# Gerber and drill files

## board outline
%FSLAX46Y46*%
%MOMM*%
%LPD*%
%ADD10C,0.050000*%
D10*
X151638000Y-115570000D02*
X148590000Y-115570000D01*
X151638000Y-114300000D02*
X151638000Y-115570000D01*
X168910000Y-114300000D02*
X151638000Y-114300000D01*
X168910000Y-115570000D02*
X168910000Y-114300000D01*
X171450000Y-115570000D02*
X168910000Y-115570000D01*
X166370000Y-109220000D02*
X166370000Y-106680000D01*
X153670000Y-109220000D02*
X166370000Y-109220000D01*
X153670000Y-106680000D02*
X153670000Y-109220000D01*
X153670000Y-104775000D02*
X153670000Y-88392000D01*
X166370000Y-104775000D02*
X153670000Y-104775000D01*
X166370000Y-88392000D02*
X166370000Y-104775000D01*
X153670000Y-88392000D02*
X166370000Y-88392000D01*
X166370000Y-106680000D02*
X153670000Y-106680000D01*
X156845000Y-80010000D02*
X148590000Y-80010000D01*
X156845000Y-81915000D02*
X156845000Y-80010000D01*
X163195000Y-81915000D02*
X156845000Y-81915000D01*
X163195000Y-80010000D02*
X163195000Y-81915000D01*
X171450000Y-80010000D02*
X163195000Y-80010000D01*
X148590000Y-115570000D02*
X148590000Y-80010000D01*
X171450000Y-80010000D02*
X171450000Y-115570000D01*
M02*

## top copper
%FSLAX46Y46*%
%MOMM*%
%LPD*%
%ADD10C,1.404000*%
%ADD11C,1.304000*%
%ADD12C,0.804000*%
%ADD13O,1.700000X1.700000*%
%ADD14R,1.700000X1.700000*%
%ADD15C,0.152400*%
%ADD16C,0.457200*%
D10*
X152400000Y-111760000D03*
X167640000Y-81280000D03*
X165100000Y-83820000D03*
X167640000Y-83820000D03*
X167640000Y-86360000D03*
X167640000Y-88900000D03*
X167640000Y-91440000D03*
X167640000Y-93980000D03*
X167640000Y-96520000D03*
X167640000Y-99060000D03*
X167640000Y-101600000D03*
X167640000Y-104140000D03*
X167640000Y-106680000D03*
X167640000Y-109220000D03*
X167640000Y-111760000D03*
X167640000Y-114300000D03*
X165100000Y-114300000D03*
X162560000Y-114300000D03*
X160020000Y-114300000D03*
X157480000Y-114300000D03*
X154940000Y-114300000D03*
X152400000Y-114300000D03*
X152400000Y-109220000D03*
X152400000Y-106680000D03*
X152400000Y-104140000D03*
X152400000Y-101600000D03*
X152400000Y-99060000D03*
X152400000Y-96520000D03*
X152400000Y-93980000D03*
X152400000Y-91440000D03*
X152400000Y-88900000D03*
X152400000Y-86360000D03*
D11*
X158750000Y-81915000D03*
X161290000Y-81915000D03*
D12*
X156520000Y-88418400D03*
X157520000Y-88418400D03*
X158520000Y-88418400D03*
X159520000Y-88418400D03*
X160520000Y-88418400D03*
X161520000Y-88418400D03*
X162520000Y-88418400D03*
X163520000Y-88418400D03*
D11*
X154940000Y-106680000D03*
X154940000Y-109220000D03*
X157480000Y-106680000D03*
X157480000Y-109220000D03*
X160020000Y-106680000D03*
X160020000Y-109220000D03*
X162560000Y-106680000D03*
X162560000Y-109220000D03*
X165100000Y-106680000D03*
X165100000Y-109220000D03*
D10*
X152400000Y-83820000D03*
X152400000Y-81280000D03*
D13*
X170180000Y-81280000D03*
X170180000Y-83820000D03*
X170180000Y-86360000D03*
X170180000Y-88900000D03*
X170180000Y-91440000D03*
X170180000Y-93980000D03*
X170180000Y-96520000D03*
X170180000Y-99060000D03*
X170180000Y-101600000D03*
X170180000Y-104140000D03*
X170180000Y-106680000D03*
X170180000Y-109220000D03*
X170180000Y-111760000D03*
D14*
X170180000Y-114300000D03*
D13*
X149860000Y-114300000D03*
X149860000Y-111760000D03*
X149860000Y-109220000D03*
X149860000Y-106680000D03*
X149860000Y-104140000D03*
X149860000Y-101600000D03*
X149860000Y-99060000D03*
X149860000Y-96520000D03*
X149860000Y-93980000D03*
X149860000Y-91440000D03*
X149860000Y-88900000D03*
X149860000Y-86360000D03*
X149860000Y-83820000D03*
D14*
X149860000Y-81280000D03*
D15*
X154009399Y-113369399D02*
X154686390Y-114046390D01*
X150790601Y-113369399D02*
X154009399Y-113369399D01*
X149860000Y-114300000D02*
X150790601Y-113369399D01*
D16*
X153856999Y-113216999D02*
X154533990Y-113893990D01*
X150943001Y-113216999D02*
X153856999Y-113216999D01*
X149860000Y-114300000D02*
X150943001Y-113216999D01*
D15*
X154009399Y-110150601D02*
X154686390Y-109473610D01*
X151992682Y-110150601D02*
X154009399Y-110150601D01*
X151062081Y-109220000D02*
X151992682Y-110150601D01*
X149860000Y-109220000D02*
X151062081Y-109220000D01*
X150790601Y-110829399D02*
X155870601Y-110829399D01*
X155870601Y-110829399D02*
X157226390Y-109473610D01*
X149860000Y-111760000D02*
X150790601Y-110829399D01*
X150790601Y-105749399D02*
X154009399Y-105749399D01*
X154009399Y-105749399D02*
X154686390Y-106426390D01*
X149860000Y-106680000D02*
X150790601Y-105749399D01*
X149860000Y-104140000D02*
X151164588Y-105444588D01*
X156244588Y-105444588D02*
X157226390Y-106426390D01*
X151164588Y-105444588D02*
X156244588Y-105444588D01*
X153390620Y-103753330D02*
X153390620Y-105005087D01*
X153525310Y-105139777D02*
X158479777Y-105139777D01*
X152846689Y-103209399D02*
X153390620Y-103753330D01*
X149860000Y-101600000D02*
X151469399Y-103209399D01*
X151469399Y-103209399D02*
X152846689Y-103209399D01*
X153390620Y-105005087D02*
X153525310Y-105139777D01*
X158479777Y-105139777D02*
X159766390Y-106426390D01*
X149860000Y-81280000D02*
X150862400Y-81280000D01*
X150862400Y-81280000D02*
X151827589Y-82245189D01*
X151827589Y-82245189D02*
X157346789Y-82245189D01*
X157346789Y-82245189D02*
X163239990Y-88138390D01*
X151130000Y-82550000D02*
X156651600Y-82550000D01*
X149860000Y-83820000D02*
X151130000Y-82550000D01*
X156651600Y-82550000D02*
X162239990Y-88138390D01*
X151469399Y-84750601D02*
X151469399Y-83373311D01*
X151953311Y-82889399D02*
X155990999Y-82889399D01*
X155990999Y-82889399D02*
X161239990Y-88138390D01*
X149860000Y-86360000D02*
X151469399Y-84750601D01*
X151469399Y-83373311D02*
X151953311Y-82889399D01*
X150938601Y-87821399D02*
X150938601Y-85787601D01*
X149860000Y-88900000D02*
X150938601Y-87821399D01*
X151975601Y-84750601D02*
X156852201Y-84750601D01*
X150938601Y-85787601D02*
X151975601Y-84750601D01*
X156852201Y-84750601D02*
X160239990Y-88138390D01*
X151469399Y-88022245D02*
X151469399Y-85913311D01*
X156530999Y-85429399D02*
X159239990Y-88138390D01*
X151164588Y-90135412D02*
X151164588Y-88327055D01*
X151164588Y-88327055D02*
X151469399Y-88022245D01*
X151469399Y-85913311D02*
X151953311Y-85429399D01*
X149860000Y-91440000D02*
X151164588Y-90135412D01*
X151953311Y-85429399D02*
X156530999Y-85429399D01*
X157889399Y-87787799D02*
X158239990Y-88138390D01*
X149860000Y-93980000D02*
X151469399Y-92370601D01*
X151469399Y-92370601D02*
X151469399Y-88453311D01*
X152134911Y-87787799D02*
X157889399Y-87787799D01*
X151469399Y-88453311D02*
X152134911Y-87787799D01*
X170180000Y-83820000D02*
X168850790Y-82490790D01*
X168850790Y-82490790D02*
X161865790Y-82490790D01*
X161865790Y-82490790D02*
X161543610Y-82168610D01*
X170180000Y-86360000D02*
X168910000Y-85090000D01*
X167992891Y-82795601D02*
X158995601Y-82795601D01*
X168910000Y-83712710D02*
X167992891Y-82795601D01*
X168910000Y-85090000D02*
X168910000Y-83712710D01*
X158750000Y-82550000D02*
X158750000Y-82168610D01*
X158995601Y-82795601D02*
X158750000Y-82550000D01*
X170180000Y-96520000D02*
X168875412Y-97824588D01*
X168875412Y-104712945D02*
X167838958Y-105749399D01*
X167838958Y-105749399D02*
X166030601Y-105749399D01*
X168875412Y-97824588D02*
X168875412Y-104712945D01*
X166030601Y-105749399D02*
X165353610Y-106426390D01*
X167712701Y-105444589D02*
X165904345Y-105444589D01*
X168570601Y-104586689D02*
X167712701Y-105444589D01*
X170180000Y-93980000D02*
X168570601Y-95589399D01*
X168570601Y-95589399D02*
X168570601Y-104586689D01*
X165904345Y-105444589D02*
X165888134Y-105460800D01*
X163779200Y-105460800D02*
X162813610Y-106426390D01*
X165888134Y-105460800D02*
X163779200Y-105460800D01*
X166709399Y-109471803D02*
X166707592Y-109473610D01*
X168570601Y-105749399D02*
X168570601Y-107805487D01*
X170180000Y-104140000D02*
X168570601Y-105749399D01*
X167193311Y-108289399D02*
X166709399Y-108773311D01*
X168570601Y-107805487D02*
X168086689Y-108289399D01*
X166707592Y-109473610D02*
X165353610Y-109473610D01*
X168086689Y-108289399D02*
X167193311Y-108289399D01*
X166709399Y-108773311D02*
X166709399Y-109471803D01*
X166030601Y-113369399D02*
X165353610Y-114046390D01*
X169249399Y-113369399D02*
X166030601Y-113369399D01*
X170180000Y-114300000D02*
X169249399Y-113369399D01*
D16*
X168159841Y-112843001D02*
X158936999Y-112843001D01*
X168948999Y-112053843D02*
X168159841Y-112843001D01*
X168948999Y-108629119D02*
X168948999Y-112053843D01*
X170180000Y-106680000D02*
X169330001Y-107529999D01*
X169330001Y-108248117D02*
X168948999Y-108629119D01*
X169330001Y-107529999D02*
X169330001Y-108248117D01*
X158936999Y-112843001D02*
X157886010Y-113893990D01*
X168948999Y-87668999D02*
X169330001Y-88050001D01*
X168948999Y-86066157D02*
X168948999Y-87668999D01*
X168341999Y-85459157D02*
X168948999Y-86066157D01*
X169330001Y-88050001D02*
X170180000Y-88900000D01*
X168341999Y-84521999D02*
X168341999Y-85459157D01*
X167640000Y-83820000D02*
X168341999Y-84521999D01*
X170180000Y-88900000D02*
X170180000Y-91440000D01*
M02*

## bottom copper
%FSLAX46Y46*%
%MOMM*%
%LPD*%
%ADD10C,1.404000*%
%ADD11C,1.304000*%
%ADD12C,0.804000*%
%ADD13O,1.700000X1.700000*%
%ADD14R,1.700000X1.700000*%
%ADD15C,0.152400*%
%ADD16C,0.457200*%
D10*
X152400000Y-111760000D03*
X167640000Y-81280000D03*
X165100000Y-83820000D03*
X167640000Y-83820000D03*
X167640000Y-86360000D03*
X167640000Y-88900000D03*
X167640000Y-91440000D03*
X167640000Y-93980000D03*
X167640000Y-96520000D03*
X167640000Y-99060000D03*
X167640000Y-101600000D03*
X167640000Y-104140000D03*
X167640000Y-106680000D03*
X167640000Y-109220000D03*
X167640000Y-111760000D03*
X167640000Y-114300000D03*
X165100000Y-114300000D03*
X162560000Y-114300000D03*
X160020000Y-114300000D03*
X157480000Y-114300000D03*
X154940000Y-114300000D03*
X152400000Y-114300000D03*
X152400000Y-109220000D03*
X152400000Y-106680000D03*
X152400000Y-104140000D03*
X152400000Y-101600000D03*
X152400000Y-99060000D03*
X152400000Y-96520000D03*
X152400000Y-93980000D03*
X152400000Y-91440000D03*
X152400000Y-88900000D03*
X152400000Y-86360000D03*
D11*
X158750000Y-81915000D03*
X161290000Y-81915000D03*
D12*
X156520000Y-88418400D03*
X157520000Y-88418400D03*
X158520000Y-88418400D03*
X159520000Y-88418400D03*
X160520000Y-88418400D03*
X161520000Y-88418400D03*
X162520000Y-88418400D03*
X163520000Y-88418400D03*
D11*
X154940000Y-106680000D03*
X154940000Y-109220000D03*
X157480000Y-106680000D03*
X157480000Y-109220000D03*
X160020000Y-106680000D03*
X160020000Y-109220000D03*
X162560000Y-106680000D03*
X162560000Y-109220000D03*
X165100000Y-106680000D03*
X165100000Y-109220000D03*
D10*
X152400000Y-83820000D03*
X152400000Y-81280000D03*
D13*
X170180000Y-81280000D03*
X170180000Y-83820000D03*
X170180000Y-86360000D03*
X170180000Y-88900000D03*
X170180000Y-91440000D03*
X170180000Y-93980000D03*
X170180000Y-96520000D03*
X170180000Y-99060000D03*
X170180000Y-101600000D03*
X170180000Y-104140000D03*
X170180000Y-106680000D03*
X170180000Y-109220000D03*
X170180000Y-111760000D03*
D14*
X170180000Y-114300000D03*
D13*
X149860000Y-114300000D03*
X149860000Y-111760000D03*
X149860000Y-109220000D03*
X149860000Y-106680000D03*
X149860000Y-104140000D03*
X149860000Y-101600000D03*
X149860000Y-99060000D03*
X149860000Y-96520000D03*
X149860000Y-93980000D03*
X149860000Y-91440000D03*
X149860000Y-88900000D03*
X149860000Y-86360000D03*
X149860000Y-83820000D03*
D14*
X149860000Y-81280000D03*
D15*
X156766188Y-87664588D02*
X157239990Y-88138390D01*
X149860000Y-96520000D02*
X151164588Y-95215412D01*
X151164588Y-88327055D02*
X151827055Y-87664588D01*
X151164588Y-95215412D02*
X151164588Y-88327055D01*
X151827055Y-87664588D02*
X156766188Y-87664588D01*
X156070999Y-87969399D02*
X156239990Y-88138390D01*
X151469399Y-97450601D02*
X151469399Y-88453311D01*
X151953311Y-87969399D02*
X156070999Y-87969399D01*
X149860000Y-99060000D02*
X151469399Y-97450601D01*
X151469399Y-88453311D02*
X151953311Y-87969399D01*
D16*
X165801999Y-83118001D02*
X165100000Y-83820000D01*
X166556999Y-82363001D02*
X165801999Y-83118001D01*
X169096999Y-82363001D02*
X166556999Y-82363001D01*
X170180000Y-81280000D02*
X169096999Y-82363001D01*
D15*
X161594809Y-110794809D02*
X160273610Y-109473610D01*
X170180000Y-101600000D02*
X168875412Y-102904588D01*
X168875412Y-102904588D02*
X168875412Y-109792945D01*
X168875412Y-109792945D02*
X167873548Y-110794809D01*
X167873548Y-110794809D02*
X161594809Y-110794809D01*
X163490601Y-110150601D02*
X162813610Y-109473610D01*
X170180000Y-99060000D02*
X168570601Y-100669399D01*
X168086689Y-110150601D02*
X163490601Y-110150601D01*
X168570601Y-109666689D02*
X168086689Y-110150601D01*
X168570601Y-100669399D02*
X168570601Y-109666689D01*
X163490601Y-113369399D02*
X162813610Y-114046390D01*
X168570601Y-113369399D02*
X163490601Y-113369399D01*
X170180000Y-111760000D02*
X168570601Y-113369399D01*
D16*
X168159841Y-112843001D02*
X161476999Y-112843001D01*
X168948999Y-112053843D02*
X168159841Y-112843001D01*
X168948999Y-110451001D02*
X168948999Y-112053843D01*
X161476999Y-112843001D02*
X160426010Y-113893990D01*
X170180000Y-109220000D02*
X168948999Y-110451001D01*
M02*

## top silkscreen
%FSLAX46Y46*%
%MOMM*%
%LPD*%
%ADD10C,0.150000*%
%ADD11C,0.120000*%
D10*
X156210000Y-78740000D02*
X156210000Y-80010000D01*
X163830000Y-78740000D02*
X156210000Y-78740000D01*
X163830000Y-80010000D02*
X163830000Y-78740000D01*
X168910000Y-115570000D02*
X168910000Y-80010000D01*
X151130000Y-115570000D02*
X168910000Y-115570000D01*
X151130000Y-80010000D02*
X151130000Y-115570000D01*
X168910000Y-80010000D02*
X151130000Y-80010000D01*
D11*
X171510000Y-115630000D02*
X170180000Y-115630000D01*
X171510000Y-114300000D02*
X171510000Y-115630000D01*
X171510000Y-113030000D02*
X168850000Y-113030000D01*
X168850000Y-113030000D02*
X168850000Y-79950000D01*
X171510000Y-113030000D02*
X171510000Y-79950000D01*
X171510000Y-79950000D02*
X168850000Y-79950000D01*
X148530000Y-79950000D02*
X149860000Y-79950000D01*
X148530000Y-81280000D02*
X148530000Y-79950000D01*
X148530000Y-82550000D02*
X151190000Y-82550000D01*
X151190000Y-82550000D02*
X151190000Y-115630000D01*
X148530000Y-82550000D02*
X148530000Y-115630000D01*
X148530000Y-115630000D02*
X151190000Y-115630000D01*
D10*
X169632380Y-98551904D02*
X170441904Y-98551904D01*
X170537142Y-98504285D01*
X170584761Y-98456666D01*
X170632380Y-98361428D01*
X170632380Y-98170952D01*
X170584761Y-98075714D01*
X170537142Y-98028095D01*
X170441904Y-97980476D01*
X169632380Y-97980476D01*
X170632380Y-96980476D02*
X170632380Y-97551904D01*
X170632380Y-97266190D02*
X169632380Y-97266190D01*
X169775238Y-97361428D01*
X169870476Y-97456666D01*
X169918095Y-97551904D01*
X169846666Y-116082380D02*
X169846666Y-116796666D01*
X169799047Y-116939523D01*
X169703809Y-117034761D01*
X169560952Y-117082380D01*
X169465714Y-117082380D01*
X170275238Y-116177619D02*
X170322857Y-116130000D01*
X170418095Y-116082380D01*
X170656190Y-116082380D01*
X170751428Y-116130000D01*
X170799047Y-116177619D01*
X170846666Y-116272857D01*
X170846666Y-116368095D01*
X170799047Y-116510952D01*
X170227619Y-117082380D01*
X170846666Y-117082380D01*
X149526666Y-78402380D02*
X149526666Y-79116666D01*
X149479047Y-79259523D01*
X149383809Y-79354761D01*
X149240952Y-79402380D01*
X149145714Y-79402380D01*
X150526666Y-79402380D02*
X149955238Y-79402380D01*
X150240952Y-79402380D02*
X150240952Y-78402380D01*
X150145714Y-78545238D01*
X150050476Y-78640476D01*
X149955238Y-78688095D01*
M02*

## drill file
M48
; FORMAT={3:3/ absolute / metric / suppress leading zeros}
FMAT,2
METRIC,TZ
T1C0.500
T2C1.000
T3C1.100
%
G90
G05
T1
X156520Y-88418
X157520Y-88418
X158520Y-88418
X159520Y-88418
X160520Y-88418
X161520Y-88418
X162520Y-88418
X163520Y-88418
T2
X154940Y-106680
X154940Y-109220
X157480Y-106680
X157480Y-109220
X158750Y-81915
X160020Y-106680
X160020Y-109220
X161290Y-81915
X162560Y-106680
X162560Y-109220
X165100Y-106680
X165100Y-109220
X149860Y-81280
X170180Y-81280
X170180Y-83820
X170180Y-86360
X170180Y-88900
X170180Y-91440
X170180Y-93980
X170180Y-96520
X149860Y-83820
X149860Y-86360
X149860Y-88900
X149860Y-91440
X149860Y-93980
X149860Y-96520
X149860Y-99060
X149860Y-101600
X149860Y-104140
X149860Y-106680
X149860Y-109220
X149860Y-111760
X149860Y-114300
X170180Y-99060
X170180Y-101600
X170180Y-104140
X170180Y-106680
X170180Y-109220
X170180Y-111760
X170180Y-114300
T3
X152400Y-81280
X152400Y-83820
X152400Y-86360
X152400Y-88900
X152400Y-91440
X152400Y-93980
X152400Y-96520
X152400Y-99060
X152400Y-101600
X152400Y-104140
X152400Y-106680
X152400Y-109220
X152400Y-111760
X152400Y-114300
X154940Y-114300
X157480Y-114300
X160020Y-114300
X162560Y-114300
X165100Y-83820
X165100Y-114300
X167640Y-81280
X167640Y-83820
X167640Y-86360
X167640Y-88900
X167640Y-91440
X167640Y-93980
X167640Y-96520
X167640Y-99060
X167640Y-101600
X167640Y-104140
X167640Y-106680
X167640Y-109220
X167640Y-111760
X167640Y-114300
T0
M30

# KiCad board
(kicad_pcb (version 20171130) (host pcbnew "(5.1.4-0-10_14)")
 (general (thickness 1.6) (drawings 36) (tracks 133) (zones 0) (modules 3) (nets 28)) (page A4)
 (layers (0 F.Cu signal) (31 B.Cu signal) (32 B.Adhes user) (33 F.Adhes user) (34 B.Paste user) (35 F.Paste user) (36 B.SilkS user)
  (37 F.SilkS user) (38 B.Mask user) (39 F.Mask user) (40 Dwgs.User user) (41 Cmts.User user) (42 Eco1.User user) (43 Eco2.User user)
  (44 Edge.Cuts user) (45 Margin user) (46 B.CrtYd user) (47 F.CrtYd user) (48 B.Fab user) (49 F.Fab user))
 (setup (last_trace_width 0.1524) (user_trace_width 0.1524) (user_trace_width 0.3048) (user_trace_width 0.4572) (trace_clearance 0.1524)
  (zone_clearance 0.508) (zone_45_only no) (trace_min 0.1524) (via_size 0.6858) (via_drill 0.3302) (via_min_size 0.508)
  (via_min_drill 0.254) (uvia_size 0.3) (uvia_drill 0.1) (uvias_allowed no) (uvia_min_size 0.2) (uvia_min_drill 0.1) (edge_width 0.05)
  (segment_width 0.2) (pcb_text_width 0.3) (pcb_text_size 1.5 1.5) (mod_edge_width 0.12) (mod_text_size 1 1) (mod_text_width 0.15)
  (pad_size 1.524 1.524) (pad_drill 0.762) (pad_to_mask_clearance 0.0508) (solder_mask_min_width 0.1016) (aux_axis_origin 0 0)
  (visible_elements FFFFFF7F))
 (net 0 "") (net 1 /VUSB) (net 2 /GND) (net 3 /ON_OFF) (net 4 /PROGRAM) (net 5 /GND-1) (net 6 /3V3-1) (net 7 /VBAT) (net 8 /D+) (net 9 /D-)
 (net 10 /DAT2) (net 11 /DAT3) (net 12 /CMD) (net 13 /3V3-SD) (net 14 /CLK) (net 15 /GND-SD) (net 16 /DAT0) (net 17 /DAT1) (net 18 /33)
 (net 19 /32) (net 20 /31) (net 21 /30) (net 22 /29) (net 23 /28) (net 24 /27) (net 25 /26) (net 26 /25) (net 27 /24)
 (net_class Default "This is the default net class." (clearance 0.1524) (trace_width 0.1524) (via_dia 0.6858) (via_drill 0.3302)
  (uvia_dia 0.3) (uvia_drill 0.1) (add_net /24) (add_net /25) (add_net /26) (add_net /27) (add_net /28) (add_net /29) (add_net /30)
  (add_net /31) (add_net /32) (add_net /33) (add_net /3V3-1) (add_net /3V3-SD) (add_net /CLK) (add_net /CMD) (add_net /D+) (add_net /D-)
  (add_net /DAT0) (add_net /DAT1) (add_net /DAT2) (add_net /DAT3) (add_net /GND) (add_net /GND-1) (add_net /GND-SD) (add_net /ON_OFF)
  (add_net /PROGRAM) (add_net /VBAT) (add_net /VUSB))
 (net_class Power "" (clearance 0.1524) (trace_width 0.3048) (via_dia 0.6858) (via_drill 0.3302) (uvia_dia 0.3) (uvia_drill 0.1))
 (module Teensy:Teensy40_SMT (layer F.Cu) (at 160.02 97.79 270)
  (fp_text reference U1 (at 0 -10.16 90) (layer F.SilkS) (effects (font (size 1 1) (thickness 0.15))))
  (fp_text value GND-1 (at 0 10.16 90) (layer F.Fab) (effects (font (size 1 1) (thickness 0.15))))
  (fp_line (start -19.05 3.81) (end -17.78 3.81) (layer F.SilkS) (width 0.15))
  (fp_line (start -19.05 -3.81) (end -19.05 3.81) (layer F.SilkS) (width 0.15))
  (fp_line (start -17.78 -3.81) (end -19.05 -3.81) (layer F.SilkS) (width 0.15))
  (fp_line (start 17.78 -8.89) (end -17.78 -8.89) (layer F.SilkS) (width 0.15))
  (fp_line (start 17.78 8.89) (end 17.78 -8.89) (layer F.SilkS) (width 0.15))
  (fp_line (start -17.78 8.89) (end 17.78 8.89) (layer F.SilkS) (width 0.15))
  (fp_line (start -17.78 -8.89) (end -17.78 8.89) (layer F.SilkS) (width 0.15))
  (pad 13 thru_hole circle (at 13.97 7.62 270) (size 1.404 1.404) (drill 1.1) (layers *.Cu *.Mask))
  (pad 33 thru_hole circle (at -16.51 -7.62 270) (size 1.404 1.404) (drill 1.1) (layers *.Cu *.Mask))
  (pad 34 thru_hole circle (at -13.97 -5.08 270) (size 1.404 1.404) (drill 1.1) (layers *.Cu *.Mask) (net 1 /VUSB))
  (pad 32 thru_hole circle (at -13.97 -7.62 270) (size 1.404 1.404) (drill 1.1) (layers *.Cu *.Mask) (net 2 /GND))
  (pad 31 thru_hole circle (at -11.43 -7.62 270) (size 1.404 1.404) (drill 1.1) (layers *.Cu *.Mask))
  (pad 30 thru_hole circle (at -8.89 -7.62 270) (size 1.404 1.404) (drill 1.1) (layers *.Cu *.Mask))
  (pad 29 thru_hole circle (at -6.35 -7.62 270) (size 1.404 1.404) (drill 1.1) (layers *.Cu *.Mask))
  (pad 28 thru_hole circle (at -3.81 -7.62 270) (size 1.404 1.404) (drill 1.1) (layers *.Cu *.Mask))
  (pad 27 thru_hole circle (at -1.27 -7.62 270) (size 1.404 1.404) (drill 1.1) (layers *.Cu *.Mask))
  (pad 26 thru_hole circle (at 1.27 -7.62 270) (size 1.404 1.404) (drill 1.1) (layers *.Cu *.Mask))
  (pad 25 thru_hole circle (at 3.81 -7.62 270) (size 1.404 1.404) (drill 1.1) (layers *.Cu *.Mask))
  (pad 24 thru_hole circle (at 6.35 -7.62 270) (size 1.404 1.404) (drill 1.1) (layers *.Cu *.Mask))
  (pad 23 thru_hole circle (at 8.89 -7.62 270) (size 1.404 1.404) (drill 1.1) (layers *.Cu *.Mask))
  (pad 22 thru_hole circle (at 11.43 -7.62 270) (size 1.404 1.404) (drill 1.1) (layers *.Cu *.Mask))
  (pad 21 thru_hole circle (at 13.97 -7.62 270) (size 1.404 1.404) (drill 1.1) (layers *.Cu *.Mask))
  (pad 20 thru_hole circle (at 16.51 -7.62 270) (size 1.404 1.404) (drill 1.1) (layers *.Cu *.Mask))
  (pad 19 thru_hole circle (at 16.51 -5.08 270) (size 1.404 1.404) (drill 1.1) (layers *.Cu *.Mask) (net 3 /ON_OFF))
  (pad 18 thru_hole circle (at 16.51 -2.54 270) (size 1.404 1.404) (drill 1.1) (layers *.Cu *.Mask) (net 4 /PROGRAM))
  (pad 17 thru_hole circle (at 16.51 0 270) (size 1.404 1.404) (drill 1.1) (layers *.Cu *.Mask) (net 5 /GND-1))
  (pad 16 thru_hole circle (at 16.51 2.54 270) (size 1.404 1.404) (drill 1.1) (layers *.Cu *.Mask) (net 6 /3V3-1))
  (pad 15 thru_hole circle (at 16.51 5.08 270) (size 1.404 1.404) (drill 1.1) (layers *.Cu *.Mask) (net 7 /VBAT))
  (pad 14 thru_hole circle (at 16.51 7.62 270) (size 1.404 1.404) (drill 1.1) (layers *.Cu *.Mask))
  (pad 12 thru_hole circle (at 11.43 7.62 270) (size 1.404 1.404) (drill 1.1) (layers *.Cu *.Mask))
  (pad 11 thru_hole circle (at 8.89 7.62 270) (size 1.404 1.404) (drill 1.1) (layers *.Cu *.Mask))
  (pad 10 thru_hole circle (at 6.35 7.62 270) (size 1.404 1.404) (drill 1.1) (layers *.Cu *.Mask))
  (pad 9 thru_hole circle (at 3.81 7.62 270) (size 1.404 1.404) (drill 1.1) (layers *.Cu *.Mask))
  (pad 8 thru_hole circle (at 1.27 7.62 270) (size 1.404 1.404) (drill 1.1) (layers *.Cu *.Mask))
  (pad 7 thru_hole circle (at -1.27 7.62 270) (size 1.404 1.404) (drill 1.1) (layers *.Cu *.Mask))
  (pad 6 thru_hole circle (at -3.81 7.62 270) (size 1.404 1.404) (drill 1.1) (layers *.Cu *.Mask))
  (pad 5 thru_hole circle (at -6.35 7.62 270) (size 1.404 1.404) (drill 1.1) (layers *.Cu *.Mask))
  (pad 4 thru_hole circle (at -8.89 7.62 270) (size 1.404 1.404) (drill 1.1) (layers *.Cu *.Mask))
  (pad 3 thru_hole circle (at -11.43 7.62 270) (size 1.404 1.404) (drill 1.1) (layers *.Cu *.Mask))
  (pad 54 thru_hole circle (at -15.875 1.27 270) (size 1.304 1.304) (drill 1) (layers *.Cu *.Mask) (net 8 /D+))
  (pad 53 thru_hole circle (at -15.875 -1.27 270) (size 1.304 1.304) (drill 1) (layers *.Cu *.Mask) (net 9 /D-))
  (pad 52 thru_hole circle (at -9.3716 3.5 270) (size 0.804 0.804) (drill 0.5) (layers *.Cu *.Mask) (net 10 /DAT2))
  (pad 51 thru_hole circle (at -9.3716 2.5 270) (size 0.804 0.804) (drill 0.5) (layers *.Cu *.Mask) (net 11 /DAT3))
  (pad 50 thru_hole circle (at -9.3716 1.5 270) (size 0.804 0.804) (drill 0.5) (layers *.Cu *.Mask) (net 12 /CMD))
  (pad 49 thru_hole circle (at -9.3716 0.5 270) (size 0.804 0.804) (drill 0.5) (layers *.Cu *.Mask) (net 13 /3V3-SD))
  (pad 48 thru_hole circle (at -9.3716 -0.5 270) (size 0.804 0.804) (drill 0.5) (layers *.Cu *.Mask) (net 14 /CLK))
  (pad 47 thru_hole circle (at -9.3716 -1.5 270) (size 0.804 0.804) (drill 0.5) (layers *.Cu *.Mask) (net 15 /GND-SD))
  (pad 46 thru_hole circle (at -9.3716 -2.5 270) (size 0.804 0.804) (drill 0.5) (layers *.Cu *.Mask) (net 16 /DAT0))
  (pad 45 thru_hole circle (at -9.3716 -3.5 270) (size 0.804 0.804) (drill 0.5) (layers *.Cu *.Mask) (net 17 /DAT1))
  (pad 44 thru_hole circle (at 8.89 5.08 270) (size 1.304 1.304) (drill 1) (layers *.Cu *.Mask) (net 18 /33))
  (pad 43 thru_hole circle (at 11.43 5.08 270) (size 1.304 1.304) (drill 1) (layers *.Cu *.Mask) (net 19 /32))
  (pad 42 thru_hole circle (at 8.89 2.54 270) (size 1.304 1.304) (drill 1) (layers *.Cu *.Mask) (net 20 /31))
  (pad 41 thru_hole circle (at 11.43 2.54 270) (size 1.304 1.304) (drill 1) (layers *.Cu *.Mask) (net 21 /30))
  (pad 40 thru_hole circle (at 8.89 0 270) (size 1.304 1.304) (drill 1) (layers *.Cu *.Mask) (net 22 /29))
  (pad 39 thru_hole circle (at 11.43 0 270) (size 1.304 1.304) (drill 1) (layers *.Cu *.Mask) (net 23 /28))
  (pad 38 thru_hole circle (at 8.89 -2.54 270) (size 1.304 1.304) (drill 1) (layers *.Cu *.Mask) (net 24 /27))
  (pad 37 thru_hole circle (at 11.43 -2.54 270) (size 1.304 1.304) (drill 1) (layers *.Cu *.Mask) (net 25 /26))
  (pad 36 thru_hole circle (at 8.89 -5.08 270) (size 1.304 1.304) (drill 1) (layers *.Cu *.Mask) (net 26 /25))
  (pad 35 thru_hole circle (at 11.43 -5.08 270) (size 1.304 1.304) (drill 1) (layers *.Cu *.Mask) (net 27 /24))
  (pad 2 thru_hole circle (at -13.97 7.62 270) (size 1.404 1.404) (drill 1.1) (layers *.Cu *.Mask))
  (pad 1 thru_hole circle (at -16.51 7.62 270) (size 1.404 1.404) (drill 1.1) (layers *.Cu *.Mask)))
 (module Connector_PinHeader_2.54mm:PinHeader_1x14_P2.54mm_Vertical (layer F.Cu) (at 170.18 114.3 180)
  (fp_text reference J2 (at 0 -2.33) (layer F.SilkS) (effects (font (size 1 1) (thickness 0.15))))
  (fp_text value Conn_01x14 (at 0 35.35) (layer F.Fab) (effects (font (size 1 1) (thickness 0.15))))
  (fp_line (start -1.33 -1.33) (end 0 -1.33) (layer F.SilkS) (width 0.12))
  (fp_line (start -1.33 0) (end -1.33 -1.33) (layer F.SilkS) (width 0.12))
  (fp_line (start -1.33 1.27) (end 1.33 1.27) (layer F.SilkS) (width 0.12))
  (fp_line (start 1.33 1.27) (end 1.33 34.35) (layer F.SilkS) (width 0.12))
  (fp_line (start -1.33 1.27) (end -1.33 34.35) (layer F.SilkS) (width 0.12))
  (fp_line (start -1.33 34.35) (end 1.33 34.35) (layer F.SilkS) (width 0.12))
  (pad 14 thru_hole oval (at 0 33.02 180) (size 1.7 1.7) (drill 1) (layers *.Cu *.Mask) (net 1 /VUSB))
  (pad 13 thru_hole oval (at 0 30.48 180) (size 1.7 1.7) (drill 1) (layers *.Cu *.Mask) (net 9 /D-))
  (pad 12 thru_hole oval (at 0 27.94 180) (size 1.7 1.7) (drill 1) (layers *.Cu *.Mask) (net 8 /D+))
  (pad 11 thru_hole oval (at 0 25.4 180) (size 1.7 1.7) (drill 1) (layers *.Cu *.Mask) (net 2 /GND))
  (pad 10 thru_hole oval (at 0 22.86 180) (size 1.7 1.7) (drill 1) (layers *.Cu *.Mask) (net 2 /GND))
  (pad 9 thru_hole oval (at 0 20.32 180) (size 1.7 1.7) (drill 1) (layers *.Cu *.Mask) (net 24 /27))
  (pad 8 thru_hole oval (at 0 17.78 180) (size 1.7 1.7) (drill 1) (layers *.Cu *.Mask) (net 26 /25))
  (pad 7 thru_hole oval (at 0 15.24 180) (size 1.7 1.7) (drill 1) (layers *.Cu *.Mask) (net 25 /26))
  (pad 6 thru_hole oval (at 0 12.7 180) (size 1.7 1.7) (drill 1) (layers *.Cu *.Mask) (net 23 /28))
  (pad 5 thru_hole oval (at 0 10.16 180) (size 1.7 1.7) (drill 1) (layers *.Cu *.Mask) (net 27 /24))
  (pad 4 thru_hole oval (at 0 7.62 180) (size 1.7 1.7) (drill 1) (layers *.Cu *.Mask) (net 6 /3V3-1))
  (pad 3 thru_hole oval (at 0 5.08 180) (size 1.7 1.7) (drill 1) (layers *.Cu *.Mask) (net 5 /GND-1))
  (pad 2 thru_hole oval (at 0 2.54 180) (size 1.7 1.7) (drill 1) (layers *.Cu *.Mask) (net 4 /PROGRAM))
  (pad 1 thru_hole rect (at 0 0 180) (size 1.7 1.7) (drill 1) (layers *.Cu *.Mask) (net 3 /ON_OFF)))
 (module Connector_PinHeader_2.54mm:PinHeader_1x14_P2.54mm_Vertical (layer F.Cu) (at 149.86 81.28)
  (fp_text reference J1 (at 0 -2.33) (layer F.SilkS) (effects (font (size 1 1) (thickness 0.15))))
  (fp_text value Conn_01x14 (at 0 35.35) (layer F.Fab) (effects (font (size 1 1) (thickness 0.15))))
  (fp_line (start -1.33 -1.33) (end 0 -1.33) (layer F.SilkS) (width 0.12))
  (fp_line (start -1.33 0) (end -1.33 -1.33) (layer F.SilkS) (width 0.12))
  (fp_line (start -1.33 1.27) (end 1.33 1.27) (layer F.SilkS) (width 0.12))
  (fp_line (start 1.33 1.27) (end 1.33 34.35) (layer F.SilkS) (width 0.12))
  (fp_line (start -1.33 1.27) (end -1.33 34.35) (layer F.SilkS) (width 0.12))
  (fp_line (start -1.33 34.35) (end 1.33 34.35) (layer F.SilkS) (width 0.12))
  (pad 14 thru_hole oval (at 0 33.02) (size 1.7 1.7) (drill 1) (layers *.Cu *.Mask) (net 7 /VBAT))
  (pad 13 thru_hole oval (at 0 30.48) (size 1.7 1.7) (drill 1) (layers *.Cu *.Mask) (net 21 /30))
  (pad 12 thru_hole oval (at 0 27.94) (size 1.7 1.7) (drill 1) (layers *.Cu *.Mask) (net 19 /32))
  (pad 11 thru_hole oval (at 0 25.4) (size 1.7 1.7) (drill 1) (layers *.Cu *.Mask) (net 18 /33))
  (pad 10 thru_hole oval (at 0 22.86) (size 1.7 1.7) (drill 1) (layers *.Cu *.Mask) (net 20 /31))
  (pad 9 thru_hole oval (at 0 20.32) (size 1.7 1.7) (drill 1) (layers *.Cu *.Mask) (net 22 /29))
  (pad 8 thru_hole oval (at 0 17.78) (size 1.7 1.7) (drill 1) (layers *.Cu *.Mask) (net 10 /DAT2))
  (pad 7 thru_hole oval (at 0 15.24) (size 1.7 1.7) (drill 1) (layers *.Cu *.Mask) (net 11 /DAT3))
  (pad 6 thru_hole oval (at 0 12.7) (size 1.7 1.7) (drill 1) (layers *.Cu *.Mask) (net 12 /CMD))
  (pad 5 thru_hole oval (at 0 10.16) (size 1.7 1.7) (drill 1) (layers *.Cu *.Mask) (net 13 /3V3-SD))
  (pad 4 thru_hole oval (at 0 7.62) (size 1.7 1.7) (drill 1) (layers *.Cu *.Mask) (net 14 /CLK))
  (pad 3 thru_hole oval (at 0 5.08) (size 1.7 1.7) (drill 1) (layers *.Cu *.Mask) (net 15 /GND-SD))
  (pad 2 thru_hole oval (at 0 2.54) (size 1.7 1.7) (drill 1) (layers *.Cu *.Mask) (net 16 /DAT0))
  (pad 1 thru_hole rect (at 0 0) (size 1.7 1.7) (drill 1) (layers *.Cu *.Mask) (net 17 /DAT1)))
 (gr_line (start 151.638 115.57) (end 148.59 115.57) (layer Edge.Cuts) (width 0.05))
 (gr_line (start 151.638 114.3) (end 151.638 115.57) (layer Edge.Cuts) (width 0.05))
 (gr_line (start 168.91 114.3) (end 151.638 114.3) (layer Edge.Cuts) (width 0.05))
 (gr_line (start 168.91 115.57) (end 168.91 114.3) (layer Edge.Cuts) (width 0.05))
 (gr_line (start 171.45 115.57) (end 168.91 115.57) (layer Edge.Cuts) (width 0.05))
 (gr_line (start 166.37 109.22) (end 166.37 106.68) (layer Edge.Cuts) (width 0.05))
 (gr_line (start 153.67 109.22) (end 166.37 109.22) (layer Edge.Cuts) (width 0.05))
 (gr_line (start 153.67 106.68) (end 153.67 109.22) (layer Edge.Cuts) (width 0.05))
 (gr_line (start 153.67 104.775) (end 153.67 88.392) (layer Edge.Cuts) (width 0.05))
 (gr_line (start 166.37 104.775) (end 153.67 104.775) (layer Edge.Cuts) (width 0.05))
 (gr_line (start 166.37 88.392) (end 166.37 104.775) (layer Edge.Cuts) (width 0.05))
 (gr_line (start 153.67 88.392) (end 166.37 88.392) (layer Edge.Cuts) (width 0.05))
 (gr_line (start 166.37 106.68) (end 153.67 106.68) (layer Edge.Cuts) (width 0.05))
 (gr_line (start 156.845 80.01) (end 148.59 80.01) (layer Edge.Cuts) (width 0.05))
 (gr_line (start 156.845 81.915) (end 156.845 80.01) (layer Edge.Cuts) (width 0.05))
 (gr_line (start 163.195 81.915) (end 156.845 81.915) (layer Edge.Cuts) (width 0.05))
 (gr_line (start 163.195 80.01) (end 163.195 81.915) (layer Edge.Cuts) (width 0.05))
 (gr_line (start 171.45 80.01) (end 163.195 80.01) (layer Edge.Cuts) (width 0.05))
 (gr_line (start 148.59 115.57) (end 148.59 80.01) (layer Edge.Cuts) (width 0.05))
 (gr_line (start 171.45 80.01) (end 171.45 115.57) (layer Edge.Cuts) (width 0.05))
 (segment (start 154.009399 113.369399) (end 154.68639 114.04639) (width 0.1524) (layer F.Cu) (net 7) (status 20))
 (segment (start 150.790601 113.369399) (end 154.009399 113.369399) (width 0.1524) (layer F.Cu) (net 7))
 (segment (start 149.86 114.3) (end 150.790601 113.369399) (width 0.1524) (layer F.Cu) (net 7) (status 10))
 (segment (start 153.856999 113.216999) (end 154.53399 113.89399) (width 0.4572) (layer F.Cu) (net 7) (status 20))
 (segment (start 150.943001 113.216999) (end 153.856999 113.216999) (width 0.4572) (layer F.Cu) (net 7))
 (segment (start 149.86 114.3) (end 150.943001 113.216999) (width 0.4572) (layer F.Cu) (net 7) (status 10))
 (segment (start 154.009399 110.150601) (end 154.68639 109.47361) (width 0.1524) (layer F.Cu) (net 19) (status 20))
 (segment (start 151.992682 110.150601) (end 154.009399 110.150601) (width 0.1524) (layer F.Cu) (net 19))
 (segment (start 151.062081 109.22) (end 151.992682 110.150601) (width 0.1524) (layer F.Cu) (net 19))
 (segment (start 149.86 109.22) (end 151.062081 109.22) (width 0.1524) (layer F.Cu) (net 19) (status 10))
 (segment (start 150.790601 110.829399) (end 155.870601 110.829399) (width 0.1524) (layer F.Cu) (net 21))
 (segment (start 155.870601 110.829399) (end 157.22639 109.47361) (width 0.1524) (layer F.Cu) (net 21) (status 20))
 (segment (start 149.86 111.76) (end 150.790601 110.829399) (width 0.1524) (layer F.Cu) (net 21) (status 10))
 (segment (start 150.790601 105.749399) (end 154.009399 105.749399) (width 0.1524) (layer F.Cu) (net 18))
 (segment (start 154.009399 105.749399) (end 154.68639 106.42639) (width 0.1524) (layer F.Cu) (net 18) (status 20))
 (segment (start 149.86 106.68) (end 150.790601 105.749399) (width 0.1524) (layer F.Cu) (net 18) (status 10))
 (segment (start 149.86 104.14) (end 151.164588 105.444588) (width 0.1524) (layer F.Cu) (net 20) (status 10))
 (segment (start 156.244588 105.444588) (end 157.22639 106.42639) (width 0.1524) (layer F.Cu) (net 20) (status 20))
 (segment (start 151.164588 105.444588) (end 156.244588 105.444588) (width 0.1524) (layer F.Cu) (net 20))
 (segment (start 153.39062 103.75333) (end 153.39062 105.005087) (width 0.1524) (layer F.Cu) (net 22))
 (segment (start 153.52531 105.139777) (end 158.479777 105.139777) (width 0.1524) (layer F.Cu) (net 22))
 (segment (start 152.846689 103.209399) (end 153.39062 103.75333) (width 0.1524) (layer F.Cu) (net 22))
 (segment (start 149.86 101.6) (end 151.469399 103.209399) (width 0.1524) (layer F.Cu) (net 22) (status 10))
 (segment (start 151.469399 103.209399) (end 152.846689 103.209399) (width 0.1524) (layer F.Cu) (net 22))
 (segment (start 153.39062 105.005087) (end 153.52531 105.139777) (width 0.1524) (layer F.Cu) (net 22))
 (segment (start 158.479777 105.139777) (end 159.76639 106.42639) (width 0.1524) (layer F.Cu) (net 22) (status 20))
 (segment (start 149.86 81.28) (end 150.8624 81.28) (width 0.1524) (layer F.Cu) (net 17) (status 10))
 (segment (start 150.8624 81.28) (end 151.827589 82.245189) (width 0.1524) (layer F.Cu) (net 17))
 (segment (start 151.827589 82.245189) (end 157.346789 82.245189) (width 0.1524) (layer F.Cu) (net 17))
 (segment (start 157.346789 82.245189) (end 163.23999 88.13839) (width 0.1524) (layer F.Cu) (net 17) (status 20))
 (segment (start 151.13 82.55) (end 156.6516 82.55) (width 0.1524) (layer F.Cu) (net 16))
 (segment (start 149.86 83.82) (end 151.13 82.55) (width 0.1524) (layer F.Cu) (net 16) (status 10))
 (segment (start 156.6516 82.55) (end 162.23999 88.13839) (width 0.1524) (layer F.Cu) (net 16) (status 20))
 (segment (start 151.469399 84.750601) (end 151.469399 83.373311) (width 0.1524) (layer F.Cu) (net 15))
 (segment (start 151.953311 82.889399) (end 155.990999 82.889399) (width 0.1524) (layer F.Cu) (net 15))
 (segment (start 155.990999 82.889399) (end 161.23999 88.13839) (width 0.1524) (layer F.Cu) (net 15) (status 20))
 (segment (start 149.86 86.36) (end 151.469399 84.750601) (width 0.1524) (layer F.Cu) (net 15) (status 10))
 (segment (start 151.469399 83.373311) (end 151.953311 82.889399) (width 0.1524) (layer F.Cu) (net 15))
 (segment (start 150.938601 87.821399) (end 150.938601 85.787601) (width 0.1524) (layer F.Cu) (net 14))
 (segment (start 149.86 88.9) (end 150.938601 87.821399) (width 0.1524) (layer F.Cu) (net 14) (status 10))
 (segment (start 151.975601 84.750601) (end 156.852201 84.750601) (width 0.1524) (layer F.Cu) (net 14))
 (segment (start 150.938601 85.787601) (end 151.975601 84.750601) (width 0.1524) (layer F.Cu) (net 14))
 (segment (start 156.852201 84.750601) (end 160.23999 88.13839) (width 0.1524) (layer F.Cu) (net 14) (status 20))
 (segment (start 151.469399 88.022245) (end 151.469399 85.913311) (width 0.1524) (layer F.Cu) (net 13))
 (segment (start 156.530999 85.429399) (end 159.23999 88.13839) (width 0.1524) (layer F.Cu) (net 13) (status 20))
 (segment (start 151.164588 90.135412) (end 151.164588 88.327055) (width 0.1524) (layer F.Cu) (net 13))
 (segment (start 151.164588 88.327055) (end 151.469399 88.022245) (width 0.1524) (layer F.Cu) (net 13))
 (segment (start 151.469399 85.913311) (end 151.953311 85.429399) (width 0.1524) (layer F.Cu) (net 13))
 (segment (start 149.86 91.44) (end 151.164588 90.135412) (width 0.1524) (layer F.Cu) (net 13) (status 10))
 (segment (start 151.953311 85.429399) (end 156.530999 85.429399) (width 0.1524) (layer F.Cu) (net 13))
 (segment (start 157.889399 87.787799) (end 158.23999 88.13839) (width 0.1524) (layer F.Cu) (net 12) (status 20))
 (segment (start 149.86 93.98) (end 151.469399 92.370601) (width 0.1524) (layer F.Cu) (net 12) (status 10))
 (segment (start 151.469399 92.370601) (end 151.469399 88.453311) (width 0.1524) (layer F.Cu) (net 12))
 (segment (start 152.134911 87.787799) (end 157.889399 87.787799) (width 0.1524) (layer F.Cu) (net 12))
 (segment (start 151.469399 88.453311) (end 152.134911 87.787799) (width 0.1524) (layer F.Cu) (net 12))
 (segment (start 156.766188 87.664588) (end 157.23999 88.13839) (width 0.1524) (layer B.Cu) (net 11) (status 20))
 (segment (start 149.86 96.52) (end 151.164588 95.215412) (width 0.1524) (layer B.Cu) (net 11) (status 10))
 (segment (start 151.164588 88.327055) (end 151.827055 87.664588) (width 0.1524) (layer B.Cu) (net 11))
 (segment (start 151.164588 95.215412) (end 151.164588 88.327055) (width 0.1524) (layer B.Cu) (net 11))
 (segment (start 151.827055 87.664588) (end 156.766188 87.664588) (width 0.1524) (layer B.Cu) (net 11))
 (segment (start 156.070999 87.969399) (end 156.23999 88.13839) (width 0.1524) (layer B.Cu) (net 10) (status 20))
 (segment (start 151.469399 97.450601) (end 151.469399 88.453311) (width 0.1524) (layer B.Cu) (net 10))
 (segment (start 151.953311 87.969399) (end 156.070999 87.969399) (width 0.1524) (layer B.Cu) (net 10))
 (segment (start 149.86 99.06) (end 151.469399 97.450601) (width 0.1524) (layer B.Cu) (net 10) (status 10))
 (segment (start 151.469399 88.453311) (end 151.953311 87.969399) (width 0.1524) (layer B.Cu) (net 10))
 (segment (start 165.801999 83.118001) (end 165.1 83.82) (width 0.4572) (layer B.Cu) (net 1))
 (segment (start 166.556999 82.363001) (end 165.801999 83.118001) (width 0.4572) (layer B.Cu) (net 1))
 (segment (start 169.096999 82.363001) (end 166.556999 82.363001) (width 0.4572) (layer B.Cu) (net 1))
 (segment (start 170.18 81.28) (end 169.096999 82.363001) (width 0.4572) (layer B.Cu) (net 1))
 (segment (start 170.18 83.82) (end 168.85079 82.49079) (width 0.1524) (layer F.Cu) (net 9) (status 10))
 (segment (start 168.85079 82.49079) (end 161.86579 82.49079) (width 0.1524) (layer F.Cu) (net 9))
 (segment (start 161.86579 82.49079) (end 161.54361 82.16861) (width 0.1524) (layer F.Cu) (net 9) (status 20))
 (segment (start 170.18 86.36) (end 168.91 85.09) (width 0.1524) (layer F.Cu) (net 8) (status 10))
 (segment (start 167.992891 82.795601) (end 158.995601 82.795601) (width 0.1524) (layer F.Cu) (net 8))
 (segment (start 168.91 83.71271) (end 167.992891 82.795601) (width 0.1524) (layer F.Cu) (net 8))
 (segment (start 168.91 85.09) (end 168.91 83.71271) (width 0.1524) (layer F.Cu) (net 8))
 (segment (start 158.75 82.55) (end 158.75 82.16861) (width 0.1524) (layer F.Cu) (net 8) (status 30))
 (segment (start 158.995601 82.795601) (end 158.75 82.55) (width 0.1524) (layer F.Cu) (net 8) (status 20))
 (segment (start 170.18 96.52) (end 168.875412 97.824588) (width 0.1524) (layer F.Cu) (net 26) (status 10))
 (segment (start 168.875412 104.712945) (end 167.838958 105.749399) (width 0.1524) (layer F.Cu) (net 26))
 (segment (start 167.838958 105.749399) (end 166.030601 105.749399) (width 0.1524) (layer F.Cu) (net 26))
 (segment (start 168.875412 97.824588) (end 168.875412 104.712945) (width 0.1524) (layer F.Cu) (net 26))
 (segment (start 166.030601 105.749399) (end 165.35361 106.42639) (width 0.1524) (layer F.Cu) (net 26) (status 20))
 (segment (start 167.712701 105.444589) (end 165.904345 105.444589) (width 0.1524) (layer F.Cu) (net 24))
 (segment (start 168.570601 104.586689) (end 167.712701 105.444589) (width 0.1524) (layer F.Cu) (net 24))
 (segment (start 170.18 93.98) (end 168.570601 95.589399) (width 0.1524) (layer F.Cu) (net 24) (status 10))
 (segment (start 168.570601 95.589399) (end 168.570601 104.586689) (width 0.1524) (layer F.Cu) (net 24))
 (segment (start 165.904345 105.444589) (end 165.888134 105.4608) (width 0.1524) (layer F.Cu) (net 24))
 (segment (start 163.7792 105.4608) (end 162.81361 106.42639) (width 0.1524) (layer F.Cu) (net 24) (status 20))
 (segment (start 165.888134 105.4608) (end 163.7792 105.4608) (width 0.1524) (layer F.Cu) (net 24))
 (segment (start 161.594809 110.794809) (end 160.27361 109.47361) (width 0.1524) (layer B.Cu) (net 23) (status 20))
 (segment (start 170.18 101.6) (end 168.875412 102.904588) (width 0.1524) (layer B.Cu) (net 23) (status 10))
 (segment (start 168.875412 102.904588) (end 168.875412 109.792945) (width 0.1524) (layer B.Cu) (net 23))
 (segment (start 168.875412 109.792945) (end 167.873548 110.794809) (width 0.1524) (layer B.Cu) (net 23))
 (segment (start 167.873548 110.794809) (end 161.594809 110.794809) (width 0.1524) (layer B.Cu) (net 23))
 (segment (start 163.490601 110.150601) (end 162.81361 109.47361) (width 0.1524) (layer B.Cu) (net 25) (status 20))
 (segment (start 170.18 99.06) (end 168.570601 100.669399) (width 0.1524) (layer B.Cu) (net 25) (status 10))
 (segment (start 168.086689 110.150601) (end 163.490601 110.150601) (width 0.1524) (layer B.Cu) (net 25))
 (segment (start 168.570601 109.666689) (end 168.086689 110.150601) (width 0.1524) (layer B.Cu) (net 25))
 (segment (start 168.570601 100.669399) (end 168.570601 109.666689) (width 0.1524) (layer B.Cu) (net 25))
 (segment (start 166.709399 109.471803) (end 166.707592 109.47361) (width 0.1524) (layer F.Cu) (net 27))
 (segment (start 168.570601 105.749399) (end 168.570601 107.805487) (width 0.1524) (layer F.Cu) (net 27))
 (segment (start 170.18 104.14) (end 168.570601 105.749399) (width 0.1524) (layer F.Cu) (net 27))
 (segment (start 167.193311 108.289399) (end 166.709399 108.773311) (width 0.1524) (layer F.Cu) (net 27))
 (segment (start 168.570601 107.805487) (end 168.086689 108.289399) (width 0.1524) (layer F.Cu) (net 27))
 (segment (start 166.707592 109.47361) (end 165.35361 109.47361) (width 0.1524) (layer F.Cu) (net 27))
 (segment (start 168.086689 108.289399) (end 167.193311 108.289399) (width 0.1524) (layer F.Cu) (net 27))
 (segment (start 166.709399 108.773311) (end 166.709399 109.471803) (width 0.1524) (layer F.Cu) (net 27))
 (segment (start 166.030601 113.369399) (end 165.35361 114.04639) (width 0.1524) (layer F.Cu) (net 3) (status 20))
 (segment (start 169.249399 113.369399) (end 166.030601 113.369399) (width 0.1524) (layer F.Cu) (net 3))
 (segment (start 170.18 114.3) (end 169.249399 113.369399) (width 0.1524) (layer F.Cu) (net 3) (status 10))
 (segment (start 163.490601 113.369399) (end 162.81361 114.04639) (width 0.1524) (layer B.Cu) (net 4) (status 20))
 (segment (start 168.570601 113.369399) (end 163.490601 113.369399) (width 0.1524) (layer B.Cu) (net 4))
 (segment (start 170.18 111.76) (end 168.570601 113.369399) (width 0.1524) (layer B.Cu) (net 4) (status 10))
 (segment (start 168.159841 112.843001) (end 161.476999 112.843001) (width 0.4572) (layer B.Cu) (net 5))
 (segment (start 168.948999 112.053843) (end 168.159841 112.843001) (width 0.4572) (layer B.Cu) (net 5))
 (segment (start 168.948999 110.451001) (end 168.948999 112.053843) (width 0.4572) (layer B.Cu) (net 5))
 (segment (start 161.476999 112.843001) (end 160.42601 113.89399) (width 0.4572) (layer B.Cu) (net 5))
 (segment (start 170.18 109.22) (end 168.948999 110.451001) (width 0.4572) (layer B.Cu) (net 5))
 (segment (start 168.159841 112.843001) (end 158.936999 112.843001) (width 0.4572) (layer F.Cu) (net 6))
 (segment (start 168.948999 112.053843) (end 168.159841 112.843001) (width 0.4572) (layer F.Cu) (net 6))
 (segment (start 168.948999 108.629119) (end 168.948999 112.053843) (width 0.4572) (layer F.Cu) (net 6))
 (segment (start 170.18 106.68) (end 169.330001 107.529999) (width 0.4572) (layer F.Cu) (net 6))
 (segment (start 169.330001 108.248117) (end 168.948999 108.629119) (width 0.4572) (layer F.Cu) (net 6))
 (segment (start 169.330001 107.529999) (end 169.330001 108.248117) (width 0.4572) (layer F.Cu) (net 6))
 (segment (start 158.936999 112.843001) (end 157.88601 113.89399) (width 0.4572) (layer F.Cu) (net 6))
 (segment (start 168.948999 87.668999) (end 169.330001 88.050001) (width 0.4572) (layer F.Cu) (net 2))
 (segment (start 168.948999 86.066157) (end 168.948999 87.668999) (width 0.4572) (layer F.Cu) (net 2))
 (segment (start 168.341999 85.459157) (end 168.948999 86.066157) (width 0.4572) (layer F.Cu) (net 2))
 (segment (start 169.330001 88.050001) (end 170.18 88.9) (width 0.4572) (layer F.Cu) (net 2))
 (segment (start 168.341999 84.521999) (end 168.341999 85.459157) (width 0.4572) (layer F.Cu) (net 2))
 (segment (start 167.64 83.82) (end 168.341999 84.521999) (width 0.4572) (layer F.Cu) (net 2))
 (segment (start 170.18 88.9) (end 170.18 91.44) (width 0.4572) (layer F.Cu) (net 2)))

